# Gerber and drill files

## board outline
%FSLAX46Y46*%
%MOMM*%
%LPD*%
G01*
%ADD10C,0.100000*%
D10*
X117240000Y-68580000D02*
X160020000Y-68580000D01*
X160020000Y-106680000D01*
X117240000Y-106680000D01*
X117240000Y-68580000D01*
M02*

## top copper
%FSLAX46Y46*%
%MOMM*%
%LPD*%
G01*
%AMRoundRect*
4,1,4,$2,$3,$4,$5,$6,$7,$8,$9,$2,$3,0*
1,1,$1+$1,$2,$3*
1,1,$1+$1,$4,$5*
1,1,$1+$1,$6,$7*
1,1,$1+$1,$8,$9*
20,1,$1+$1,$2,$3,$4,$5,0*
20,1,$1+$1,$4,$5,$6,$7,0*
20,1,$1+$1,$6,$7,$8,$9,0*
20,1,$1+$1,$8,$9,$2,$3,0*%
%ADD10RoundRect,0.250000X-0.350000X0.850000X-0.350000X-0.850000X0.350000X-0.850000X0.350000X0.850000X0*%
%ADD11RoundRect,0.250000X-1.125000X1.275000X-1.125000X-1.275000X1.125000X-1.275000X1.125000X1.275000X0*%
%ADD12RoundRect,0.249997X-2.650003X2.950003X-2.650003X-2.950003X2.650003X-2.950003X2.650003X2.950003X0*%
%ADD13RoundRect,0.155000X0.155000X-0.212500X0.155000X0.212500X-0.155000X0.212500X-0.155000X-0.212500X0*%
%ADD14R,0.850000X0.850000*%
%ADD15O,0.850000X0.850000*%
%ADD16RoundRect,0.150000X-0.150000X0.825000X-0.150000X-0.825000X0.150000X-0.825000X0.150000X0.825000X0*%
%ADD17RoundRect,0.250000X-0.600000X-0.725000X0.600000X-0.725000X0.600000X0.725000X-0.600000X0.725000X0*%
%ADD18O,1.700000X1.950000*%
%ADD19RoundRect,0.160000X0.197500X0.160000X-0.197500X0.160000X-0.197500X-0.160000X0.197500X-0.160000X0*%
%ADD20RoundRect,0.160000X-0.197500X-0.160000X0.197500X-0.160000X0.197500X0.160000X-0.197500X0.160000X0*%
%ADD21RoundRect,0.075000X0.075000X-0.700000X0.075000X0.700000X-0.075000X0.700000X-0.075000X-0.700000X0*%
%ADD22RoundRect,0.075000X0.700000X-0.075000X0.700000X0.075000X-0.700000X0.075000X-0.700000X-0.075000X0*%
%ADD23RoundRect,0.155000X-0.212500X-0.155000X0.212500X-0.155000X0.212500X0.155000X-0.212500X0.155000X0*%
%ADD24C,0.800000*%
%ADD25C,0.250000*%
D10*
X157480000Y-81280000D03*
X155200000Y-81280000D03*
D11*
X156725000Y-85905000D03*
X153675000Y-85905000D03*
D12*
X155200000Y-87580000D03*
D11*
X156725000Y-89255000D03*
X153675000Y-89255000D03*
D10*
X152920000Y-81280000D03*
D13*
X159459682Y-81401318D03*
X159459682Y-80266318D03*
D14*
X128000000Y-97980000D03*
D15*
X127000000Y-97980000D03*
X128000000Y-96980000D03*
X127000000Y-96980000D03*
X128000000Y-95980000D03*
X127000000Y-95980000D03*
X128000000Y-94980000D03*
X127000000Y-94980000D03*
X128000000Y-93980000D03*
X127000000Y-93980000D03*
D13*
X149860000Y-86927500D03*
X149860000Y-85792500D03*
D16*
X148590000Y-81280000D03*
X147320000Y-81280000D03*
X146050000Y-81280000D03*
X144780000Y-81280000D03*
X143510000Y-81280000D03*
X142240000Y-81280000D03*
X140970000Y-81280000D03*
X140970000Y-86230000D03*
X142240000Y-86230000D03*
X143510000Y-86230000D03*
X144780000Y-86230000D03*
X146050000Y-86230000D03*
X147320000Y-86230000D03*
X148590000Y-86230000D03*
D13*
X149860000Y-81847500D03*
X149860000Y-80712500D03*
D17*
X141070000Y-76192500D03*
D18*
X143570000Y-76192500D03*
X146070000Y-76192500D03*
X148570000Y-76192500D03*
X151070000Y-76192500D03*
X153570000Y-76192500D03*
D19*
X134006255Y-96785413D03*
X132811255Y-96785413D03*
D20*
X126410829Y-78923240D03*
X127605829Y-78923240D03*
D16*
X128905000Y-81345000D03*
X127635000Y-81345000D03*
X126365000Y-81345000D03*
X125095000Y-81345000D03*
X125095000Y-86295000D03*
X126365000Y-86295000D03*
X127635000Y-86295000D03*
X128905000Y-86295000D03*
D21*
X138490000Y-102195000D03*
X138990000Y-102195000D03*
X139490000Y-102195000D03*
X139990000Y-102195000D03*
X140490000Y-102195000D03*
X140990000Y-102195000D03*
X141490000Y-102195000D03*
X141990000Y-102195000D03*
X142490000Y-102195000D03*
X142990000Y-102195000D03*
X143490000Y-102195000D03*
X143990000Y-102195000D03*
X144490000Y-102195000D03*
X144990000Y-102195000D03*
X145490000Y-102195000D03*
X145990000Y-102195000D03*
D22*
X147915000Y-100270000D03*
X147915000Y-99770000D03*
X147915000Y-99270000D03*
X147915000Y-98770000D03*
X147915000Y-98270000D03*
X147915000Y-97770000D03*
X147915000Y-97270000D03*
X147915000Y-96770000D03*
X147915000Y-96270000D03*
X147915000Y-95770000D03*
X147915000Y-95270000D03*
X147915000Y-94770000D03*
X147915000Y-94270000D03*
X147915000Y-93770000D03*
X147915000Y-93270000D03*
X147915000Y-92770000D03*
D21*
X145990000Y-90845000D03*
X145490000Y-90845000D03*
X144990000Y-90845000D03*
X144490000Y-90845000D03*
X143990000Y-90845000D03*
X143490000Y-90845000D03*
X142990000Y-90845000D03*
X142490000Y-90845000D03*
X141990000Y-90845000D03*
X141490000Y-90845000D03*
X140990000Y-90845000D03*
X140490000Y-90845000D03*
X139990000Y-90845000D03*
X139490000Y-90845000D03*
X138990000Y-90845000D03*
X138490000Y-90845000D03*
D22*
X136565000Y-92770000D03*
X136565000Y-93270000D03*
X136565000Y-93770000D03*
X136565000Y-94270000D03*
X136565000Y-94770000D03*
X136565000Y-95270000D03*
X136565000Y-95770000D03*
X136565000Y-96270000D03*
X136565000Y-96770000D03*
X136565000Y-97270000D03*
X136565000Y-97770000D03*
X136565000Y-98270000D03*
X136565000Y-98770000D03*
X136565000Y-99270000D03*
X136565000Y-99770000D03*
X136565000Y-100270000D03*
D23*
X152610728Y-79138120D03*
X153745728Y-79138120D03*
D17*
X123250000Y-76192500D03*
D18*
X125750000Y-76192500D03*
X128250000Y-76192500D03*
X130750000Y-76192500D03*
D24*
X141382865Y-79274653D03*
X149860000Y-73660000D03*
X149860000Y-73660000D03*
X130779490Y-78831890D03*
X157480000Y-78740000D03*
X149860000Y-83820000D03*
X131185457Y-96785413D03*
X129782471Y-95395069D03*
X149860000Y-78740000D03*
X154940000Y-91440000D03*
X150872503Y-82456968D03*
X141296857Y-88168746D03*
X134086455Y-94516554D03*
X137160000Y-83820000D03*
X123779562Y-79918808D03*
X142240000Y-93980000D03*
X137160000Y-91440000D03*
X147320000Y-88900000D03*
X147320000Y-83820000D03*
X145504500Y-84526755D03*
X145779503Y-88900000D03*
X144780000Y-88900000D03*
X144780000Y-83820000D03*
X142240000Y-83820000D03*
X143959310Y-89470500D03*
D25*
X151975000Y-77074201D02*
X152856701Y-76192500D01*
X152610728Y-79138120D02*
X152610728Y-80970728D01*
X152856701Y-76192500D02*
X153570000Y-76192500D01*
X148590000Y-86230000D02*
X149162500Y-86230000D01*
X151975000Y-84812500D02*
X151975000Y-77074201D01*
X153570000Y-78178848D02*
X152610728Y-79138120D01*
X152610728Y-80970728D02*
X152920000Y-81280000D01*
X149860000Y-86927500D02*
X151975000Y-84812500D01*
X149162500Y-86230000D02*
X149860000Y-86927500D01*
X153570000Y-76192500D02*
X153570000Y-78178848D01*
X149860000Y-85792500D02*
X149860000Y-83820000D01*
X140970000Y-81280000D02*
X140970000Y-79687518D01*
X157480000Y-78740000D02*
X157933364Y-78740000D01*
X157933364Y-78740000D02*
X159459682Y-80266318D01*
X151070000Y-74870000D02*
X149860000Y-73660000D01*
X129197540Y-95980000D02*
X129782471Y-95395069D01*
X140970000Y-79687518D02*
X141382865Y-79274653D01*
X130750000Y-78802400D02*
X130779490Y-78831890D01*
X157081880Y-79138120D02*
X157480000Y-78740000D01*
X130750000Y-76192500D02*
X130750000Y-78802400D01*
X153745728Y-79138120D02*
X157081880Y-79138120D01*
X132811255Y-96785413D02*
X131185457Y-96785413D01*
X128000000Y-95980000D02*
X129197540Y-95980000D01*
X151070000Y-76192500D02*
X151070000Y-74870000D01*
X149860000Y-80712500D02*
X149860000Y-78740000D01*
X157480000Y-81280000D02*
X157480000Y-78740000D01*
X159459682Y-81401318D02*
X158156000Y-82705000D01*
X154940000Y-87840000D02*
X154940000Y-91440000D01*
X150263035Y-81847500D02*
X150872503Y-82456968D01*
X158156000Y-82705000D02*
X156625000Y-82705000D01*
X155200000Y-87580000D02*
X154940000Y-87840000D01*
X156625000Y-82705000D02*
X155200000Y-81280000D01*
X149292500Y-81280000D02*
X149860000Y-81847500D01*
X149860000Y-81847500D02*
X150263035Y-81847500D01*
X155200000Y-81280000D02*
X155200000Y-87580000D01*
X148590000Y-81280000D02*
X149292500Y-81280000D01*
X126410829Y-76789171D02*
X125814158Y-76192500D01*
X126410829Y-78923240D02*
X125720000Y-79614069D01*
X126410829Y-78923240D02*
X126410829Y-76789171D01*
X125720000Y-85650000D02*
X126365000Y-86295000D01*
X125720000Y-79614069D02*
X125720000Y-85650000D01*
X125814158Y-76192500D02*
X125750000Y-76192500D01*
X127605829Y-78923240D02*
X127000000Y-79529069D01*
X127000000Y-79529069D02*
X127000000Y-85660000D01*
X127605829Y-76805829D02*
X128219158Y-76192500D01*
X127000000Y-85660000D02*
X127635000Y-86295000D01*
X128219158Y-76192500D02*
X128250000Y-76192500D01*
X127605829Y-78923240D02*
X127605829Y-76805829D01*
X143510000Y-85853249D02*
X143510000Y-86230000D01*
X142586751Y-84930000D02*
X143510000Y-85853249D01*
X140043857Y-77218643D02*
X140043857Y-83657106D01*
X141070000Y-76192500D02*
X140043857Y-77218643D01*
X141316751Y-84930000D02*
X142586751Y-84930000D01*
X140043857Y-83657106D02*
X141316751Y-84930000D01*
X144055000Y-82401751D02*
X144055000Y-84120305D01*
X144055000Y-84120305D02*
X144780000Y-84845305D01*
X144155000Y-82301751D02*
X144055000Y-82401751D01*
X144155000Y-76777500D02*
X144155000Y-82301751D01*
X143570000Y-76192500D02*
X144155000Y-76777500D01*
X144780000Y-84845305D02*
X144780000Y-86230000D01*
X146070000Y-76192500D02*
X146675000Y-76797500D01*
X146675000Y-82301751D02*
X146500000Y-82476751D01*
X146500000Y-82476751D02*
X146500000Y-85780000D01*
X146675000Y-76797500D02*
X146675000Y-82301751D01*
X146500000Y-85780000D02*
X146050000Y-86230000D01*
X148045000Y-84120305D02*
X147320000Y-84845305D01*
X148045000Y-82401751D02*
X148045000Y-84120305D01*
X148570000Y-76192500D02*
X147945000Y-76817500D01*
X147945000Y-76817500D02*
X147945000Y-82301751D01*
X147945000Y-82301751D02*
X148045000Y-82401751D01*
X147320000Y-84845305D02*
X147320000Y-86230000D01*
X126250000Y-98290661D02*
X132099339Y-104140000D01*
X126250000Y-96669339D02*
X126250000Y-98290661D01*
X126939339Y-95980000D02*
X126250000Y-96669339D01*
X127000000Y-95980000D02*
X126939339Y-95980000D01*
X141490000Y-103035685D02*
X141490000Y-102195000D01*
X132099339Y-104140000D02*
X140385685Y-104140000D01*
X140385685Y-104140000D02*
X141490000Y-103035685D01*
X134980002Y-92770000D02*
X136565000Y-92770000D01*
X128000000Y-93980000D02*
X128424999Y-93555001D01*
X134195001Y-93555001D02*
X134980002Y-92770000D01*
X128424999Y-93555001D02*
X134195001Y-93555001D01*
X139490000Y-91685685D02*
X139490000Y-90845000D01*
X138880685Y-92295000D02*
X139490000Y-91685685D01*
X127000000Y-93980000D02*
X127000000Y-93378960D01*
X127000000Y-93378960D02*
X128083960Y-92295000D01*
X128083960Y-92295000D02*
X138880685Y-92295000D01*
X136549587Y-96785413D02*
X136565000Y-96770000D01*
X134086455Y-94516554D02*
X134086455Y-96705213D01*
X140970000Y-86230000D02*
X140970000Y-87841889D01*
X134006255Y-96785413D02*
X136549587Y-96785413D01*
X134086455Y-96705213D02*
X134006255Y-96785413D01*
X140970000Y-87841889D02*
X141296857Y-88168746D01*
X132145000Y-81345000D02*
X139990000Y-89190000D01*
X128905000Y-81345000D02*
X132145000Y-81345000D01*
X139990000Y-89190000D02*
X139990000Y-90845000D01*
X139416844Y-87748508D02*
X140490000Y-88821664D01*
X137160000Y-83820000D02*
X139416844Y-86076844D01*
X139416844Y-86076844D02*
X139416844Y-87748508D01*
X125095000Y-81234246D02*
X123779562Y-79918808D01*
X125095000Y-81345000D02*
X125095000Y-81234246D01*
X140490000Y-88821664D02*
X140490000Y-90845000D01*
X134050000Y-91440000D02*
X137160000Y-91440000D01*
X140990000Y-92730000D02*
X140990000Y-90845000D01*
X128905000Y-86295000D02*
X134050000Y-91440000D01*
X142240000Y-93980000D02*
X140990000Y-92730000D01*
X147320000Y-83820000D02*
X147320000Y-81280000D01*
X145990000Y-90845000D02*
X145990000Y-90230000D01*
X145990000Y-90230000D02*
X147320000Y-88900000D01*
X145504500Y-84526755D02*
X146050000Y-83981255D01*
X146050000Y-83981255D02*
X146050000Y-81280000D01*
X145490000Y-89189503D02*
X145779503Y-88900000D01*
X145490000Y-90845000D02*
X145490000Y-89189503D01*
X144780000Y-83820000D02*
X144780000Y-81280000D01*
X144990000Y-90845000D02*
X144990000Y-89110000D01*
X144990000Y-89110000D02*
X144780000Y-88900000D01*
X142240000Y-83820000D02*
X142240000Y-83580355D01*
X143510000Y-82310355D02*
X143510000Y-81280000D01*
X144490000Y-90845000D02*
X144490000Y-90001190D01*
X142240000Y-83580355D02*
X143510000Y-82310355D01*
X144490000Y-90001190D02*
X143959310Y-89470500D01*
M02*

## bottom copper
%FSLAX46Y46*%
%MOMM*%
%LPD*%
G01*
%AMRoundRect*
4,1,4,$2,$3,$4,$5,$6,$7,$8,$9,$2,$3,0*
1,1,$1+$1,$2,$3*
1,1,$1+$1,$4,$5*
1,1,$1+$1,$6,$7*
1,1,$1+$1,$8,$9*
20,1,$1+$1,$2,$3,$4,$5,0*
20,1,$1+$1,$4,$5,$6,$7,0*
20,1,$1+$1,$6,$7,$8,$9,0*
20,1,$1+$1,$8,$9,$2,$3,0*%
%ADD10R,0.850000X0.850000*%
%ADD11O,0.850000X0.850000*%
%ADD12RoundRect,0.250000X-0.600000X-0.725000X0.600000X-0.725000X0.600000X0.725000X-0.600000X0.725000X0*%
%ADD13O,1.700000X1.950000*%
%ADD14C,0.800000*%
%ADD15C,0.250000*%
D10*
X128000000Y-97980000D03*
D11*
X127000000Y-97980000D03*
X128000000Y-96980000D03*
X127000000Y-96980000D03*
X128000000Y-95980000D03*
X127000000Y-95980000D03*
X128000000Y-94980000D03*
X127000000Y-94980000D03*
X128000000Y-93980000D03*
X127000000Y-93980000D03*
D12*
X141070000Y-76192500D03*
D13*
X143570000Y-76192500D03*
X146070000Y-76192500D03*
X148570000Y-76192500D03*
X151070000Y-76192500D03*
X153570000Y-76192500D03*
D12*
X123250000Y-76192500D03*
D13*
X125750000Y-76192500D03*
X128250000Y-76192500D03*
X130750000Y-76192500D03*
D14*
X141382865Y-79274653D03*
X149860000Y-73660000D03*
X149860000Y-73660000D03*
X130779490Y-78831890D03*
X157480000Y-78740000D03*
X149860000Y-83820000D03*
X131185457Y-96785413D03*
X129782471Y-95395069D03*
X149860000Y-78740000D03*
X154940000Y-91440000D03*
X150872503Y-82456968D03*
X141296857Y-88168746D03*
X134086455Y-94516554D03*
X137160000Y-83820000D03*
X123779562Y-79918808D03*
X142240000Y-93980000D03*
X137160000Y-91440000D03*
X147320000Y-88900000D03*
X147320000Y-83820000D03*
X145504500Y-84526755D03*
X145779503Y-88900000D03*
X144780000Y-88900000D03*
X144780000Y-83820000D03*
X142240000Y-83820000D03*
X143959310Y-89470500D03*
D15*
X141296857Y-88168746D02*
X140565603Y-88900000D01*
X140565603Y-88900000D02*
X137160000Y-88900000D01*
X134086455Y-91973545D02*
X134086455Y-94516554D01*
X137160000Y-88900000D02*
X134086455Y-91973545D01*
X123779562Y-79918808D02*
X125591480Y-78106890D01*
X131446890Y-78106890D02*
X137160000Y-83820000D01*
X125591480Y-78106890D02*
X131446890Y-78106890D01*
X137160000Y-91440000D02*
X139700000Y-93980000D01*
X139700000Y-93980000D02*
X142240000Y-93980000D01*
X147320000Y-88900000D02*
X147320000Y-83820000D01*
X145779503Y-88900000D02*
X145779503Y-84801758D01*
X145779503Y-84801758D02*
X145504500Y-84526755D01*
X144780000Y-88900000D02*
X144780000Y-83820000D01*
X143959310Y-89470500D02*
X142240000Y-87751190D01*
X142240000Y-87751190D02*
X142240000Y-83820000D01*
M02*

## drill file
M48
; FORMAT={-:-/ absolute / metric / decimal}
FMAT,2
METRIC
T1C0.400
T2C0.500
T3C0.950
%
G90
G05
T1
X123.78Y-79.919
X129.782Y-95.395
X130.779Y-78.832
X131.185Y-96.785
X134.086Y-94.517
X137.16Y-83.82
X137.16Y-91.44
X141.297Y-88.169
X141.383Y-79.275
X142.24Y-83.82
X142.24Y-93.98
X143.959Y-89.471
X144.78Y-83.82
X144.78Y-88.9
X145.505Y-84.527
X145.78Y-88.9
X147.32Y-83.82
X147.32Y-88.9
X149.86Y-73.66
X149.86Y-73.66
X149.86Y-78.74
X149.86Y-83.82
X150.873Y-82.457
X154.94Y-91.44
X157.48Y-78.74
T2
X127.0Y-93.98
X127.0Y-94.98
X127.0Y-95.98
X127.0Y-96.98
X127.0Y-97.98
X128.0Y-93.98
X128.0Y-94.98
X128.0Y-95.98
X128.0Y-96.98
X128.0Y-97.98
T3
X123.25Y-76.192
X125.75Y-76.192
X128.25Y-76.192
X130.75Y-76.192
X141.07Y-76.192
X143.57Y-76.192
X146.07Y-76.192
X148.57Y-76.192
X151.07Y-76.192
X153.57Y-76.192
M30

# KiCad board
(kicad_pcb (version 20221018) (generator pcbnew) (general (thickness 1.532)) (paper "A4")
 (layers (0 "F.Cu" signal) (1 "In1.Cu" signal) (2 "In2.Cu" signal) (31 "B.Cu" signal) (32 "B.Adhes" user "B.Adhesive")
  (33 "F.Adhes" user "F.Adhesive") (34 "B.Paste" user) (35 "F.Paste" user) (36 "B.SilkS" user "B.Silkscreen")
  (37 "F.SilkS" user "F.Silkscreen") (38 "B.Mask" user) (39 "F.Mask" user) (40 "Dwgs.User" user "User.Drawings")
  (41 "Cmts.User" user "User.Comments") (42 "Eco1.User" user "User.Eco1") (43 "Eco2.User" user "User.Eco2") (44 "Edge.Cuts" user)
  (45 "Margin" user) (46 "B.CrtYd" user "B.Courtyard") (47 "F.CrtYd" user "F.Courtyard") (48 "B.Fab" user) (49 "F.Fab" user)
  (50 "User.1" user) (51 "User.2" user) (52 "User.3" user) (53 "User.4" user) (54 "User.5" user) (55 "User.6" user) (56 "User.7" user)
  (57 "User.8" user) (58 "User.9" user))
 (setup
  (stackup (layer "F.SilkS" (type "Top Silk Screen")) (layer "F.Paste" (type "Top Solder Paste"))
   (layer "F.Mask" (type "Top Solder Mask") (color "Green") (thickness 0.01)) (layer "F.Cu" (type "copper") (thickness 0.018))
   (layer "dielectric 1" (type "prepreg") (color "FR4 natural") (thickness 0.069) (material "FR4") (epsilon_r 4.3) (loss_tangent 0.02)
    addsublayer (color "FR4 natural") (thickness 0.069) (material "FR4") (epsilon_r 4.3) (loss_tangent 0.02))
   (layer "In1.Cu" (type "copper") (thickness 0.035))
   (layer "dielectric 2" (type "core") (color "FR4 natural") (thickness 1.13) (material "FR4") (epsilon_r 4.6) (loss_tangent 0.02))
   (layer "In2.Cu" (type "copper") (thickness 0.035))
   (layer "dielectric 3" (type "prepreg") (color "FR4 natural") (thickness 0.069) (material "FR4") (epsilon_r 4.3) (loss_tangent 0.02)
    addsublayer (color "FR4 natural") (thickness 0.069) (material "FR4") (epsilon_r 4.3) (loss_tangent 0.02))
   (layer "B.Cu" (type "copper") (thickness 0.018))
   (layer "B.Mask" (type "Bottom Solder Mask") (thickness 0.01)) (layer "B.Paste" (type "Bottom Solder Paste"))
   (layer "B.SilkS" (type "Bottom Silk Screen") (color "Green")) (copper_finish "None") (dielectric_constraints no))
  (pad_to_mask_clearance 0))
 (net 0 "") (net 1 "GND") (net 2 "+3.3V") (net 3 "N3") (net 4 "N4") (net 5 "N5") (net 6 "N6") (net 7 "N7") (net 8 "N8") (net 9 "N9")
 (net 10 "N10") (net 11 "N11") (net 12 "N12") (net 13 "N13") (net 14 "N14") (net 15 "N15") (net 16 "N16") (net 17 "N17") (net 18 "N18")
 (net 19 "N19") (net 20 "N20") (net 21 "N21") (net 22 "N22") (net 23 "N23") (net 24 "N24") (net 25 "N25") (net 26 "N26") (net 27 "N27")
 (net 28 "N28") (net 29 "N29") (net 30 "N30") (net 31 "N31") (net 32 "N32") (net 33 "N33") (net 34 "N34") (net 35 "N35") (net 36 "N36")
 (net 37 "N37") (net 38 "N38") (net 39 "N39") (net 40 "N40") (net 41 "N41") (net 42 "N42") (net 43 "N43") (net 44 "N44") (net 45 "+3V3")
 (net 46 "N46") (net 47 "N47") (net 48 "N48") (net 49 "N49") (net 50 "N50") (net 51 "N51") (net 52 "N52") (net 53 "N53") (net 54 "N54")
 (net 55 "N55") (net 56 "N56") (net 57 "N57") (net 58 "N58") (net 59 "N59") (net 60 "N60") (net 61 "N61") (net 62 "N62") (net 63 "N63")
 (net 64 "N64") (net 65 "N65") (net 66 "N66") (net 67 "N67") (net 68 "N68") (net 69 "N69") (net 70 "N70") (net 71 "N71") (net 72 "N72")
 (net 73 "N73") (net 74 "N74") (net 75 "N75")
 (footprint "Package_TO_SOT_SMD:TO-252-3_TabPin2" (layer "F.Cu") (at 155.2 86.32 -90)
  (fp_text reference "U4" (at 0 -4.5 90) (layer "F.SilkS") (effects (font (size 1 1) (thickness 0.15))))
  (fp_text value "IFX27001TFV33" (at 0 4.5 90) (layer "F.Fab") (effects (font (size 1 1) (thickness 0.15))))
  (pad "1" smd roundrect (at -5.04 -2.28 270) (size 2.2 1.2) (layers "F.Cu" "F.Paste" "F.Mask") (roundrect_rratio 0.208333) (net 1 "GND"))
  (pad "2" smd roundrect (at -5.04 0 270) (size 2.2 1.2) (layers "F.Cu" "F.Paste" "F.Mask") (roundrect_rratio 0.208333) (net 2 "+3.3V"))
  (pad "2" smd roundrect (at -0.415 -1.525 270) (size 3.05 2.75) (layers "F.Cu" "F.Paste") (roundrect_rratio 0.090909) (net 2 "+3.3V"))
  (pad "2" smd roundrect (at -0.415 1.525 270) (size 3.05 2.75) (layers "F.Cu" "F.Paste") (roundrect_rratio 0.090909) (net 2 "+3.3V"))
  (pad "2" smd roundrect (at 1.26 0 270) (size 6.4 5.8) (layers "F.Cu" "F.Mask") (roundrect_rratio 0.043103) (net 2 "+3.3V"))
  (pad "2" smd roundrect (at 2.935 -1.525 270) (size 3.05 2.75) (layers "F.Cu" "F.Paste") (roundrect_rratio 0.090909) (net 2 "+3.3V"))
  (pad "2" smd roundrect (at 2.935 1.525 270) (size 3.05 2.75) (layers "F.Cu" "F.Paste") (roundrect_rratio 0.090909) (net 2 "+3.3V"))
  (pad "3" smd roundrect (at -5.04 2.28 270) (size 2.2 1.2) (layers "F.Cu" "F.Paste" "F.Mask") (roundrect_rratio 0.208333) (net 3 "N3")))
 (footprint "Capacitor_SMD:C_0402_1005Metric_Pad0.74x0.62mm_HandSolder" (layer "F.Cu") (at 159.459682 80.833818 90)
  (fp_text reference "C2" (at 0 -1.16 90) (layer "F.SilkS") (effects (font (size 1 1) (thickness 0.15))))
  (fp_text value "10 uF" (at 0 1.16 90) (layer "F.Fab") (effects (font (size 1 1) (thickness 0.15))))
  (pad "1" smd roundrect (at -0.5675 0 90) (size 0.735 0.62) (layers "F.Cu" "F.Paste" "F.Mask") (roundrect_rratio 0.25) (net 2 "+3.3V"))
  (pad "2" smd roundrect (at 0.5675 0 90) (size 0.735 0.62) (layers "F.Cu" "F.Paste" "F.Mask") (roundrect_rratio 0.25) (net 1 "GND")))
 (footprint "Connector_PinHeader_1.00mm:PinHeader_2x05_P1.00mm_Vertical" (layer "F.Cu") (at 128 97.98 180)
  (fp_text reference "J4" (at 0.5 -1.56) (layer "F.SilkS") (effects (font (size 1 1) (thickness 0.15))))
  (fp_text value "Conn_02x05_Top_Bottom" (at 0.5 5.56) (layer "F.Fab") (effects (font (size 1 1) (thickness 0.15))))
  (pad "1" thru_hole rect (at 0 0 180) (size 0.85 0.85) (drill 0.5) (layers "*.Cu" "*.Mask") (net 2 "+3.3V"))
  (pad "2" thru_hole oval (at 1 0 180) (size 0.85 0.85) (drill 0.5) (layers "*.Cu" "*.Mask") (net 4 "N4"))
  (pad "3" thru_hole oval (at 0 1 180) (size 0.85 0.85) (drill 0.5) (layers "*.Cu" "*.Mask") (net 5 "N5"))
  (pad "4" thru_hole oval (at 1 1 180) (size 0.85 0.85) (drill 0.5) (layers "*.Cu" "*.Mask") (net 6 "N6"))
  (pad "5" thru_hole oval (at 0 2 180) (size 0.85 0.85) (drill 0.5) (layers "*.Cu" "*.Mask") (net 1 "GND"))
  (pad "6" thru_hole oval (at 1 2 180) (size 0.85 0.85) (drill 0.5) (layers "*.Cu" "*.Mask") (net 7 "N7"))
  (pad "7" thru_hole oval (at 0 3 180) (size 0.85 0.85) (drill 0.5) (layers "*.Cu" "*.Mask") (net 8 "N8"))
  (pad "8" thru_hole oval (at 1 3 180) (size 0.85 0.85) (drill 0.5) (layers "*.Cu" "*.Mask") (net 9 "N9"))
  (pad "9" thru_hole oval (at 0 4 180) (size 0.85 0.85) (drill 0.5) (layers "*.Cu" "*.Mask") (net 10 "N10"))
  (pad "10" thru_hole oval (at 1 4 180) (size 0.85 0.85) (drill 0.5) (layers "*.Cu" "*.Mask") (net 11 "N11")))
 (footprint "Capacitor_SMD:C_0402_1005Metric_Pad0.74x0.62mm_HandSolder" (layer "F.Cu") (at 149.86 86.36 90)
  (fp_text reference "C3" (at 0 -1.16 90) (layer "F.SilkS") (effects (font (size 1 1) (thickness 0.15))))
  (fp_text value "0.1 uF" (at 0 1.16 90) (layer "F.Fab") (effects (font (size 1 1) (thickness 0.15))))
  (pad "1" smd roundrect (at -0.5675 0 90) (size 0.735 0.62) (layers "F.Cu" "F.Paste" "F.Mask") (roundrect_rratio 0.25) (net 3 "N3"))
  (pad "2" smd roundrect (at 0.5675 0 90) (size 0.735 0.62) (layers "F.Cu" "F.Paste" "F.Mask") (roundrect_rratio 0.25) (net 1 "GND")))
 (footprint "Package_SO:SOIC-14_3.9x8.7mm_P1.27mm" (layer "F.Cu") (at 144.78 83.755 -90)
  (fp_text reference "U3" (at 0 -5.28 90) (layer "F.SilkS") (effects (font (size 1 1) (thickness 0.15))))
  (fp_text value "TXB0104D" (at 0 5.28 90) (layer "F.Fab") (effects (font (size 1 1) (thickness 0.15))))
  (pad "1" smd roundrect (at -2.475 -3.81 270) (size 1.95 0.6) (layers "F.Cu" "F.Paste" "F.Mask") (roundrect_rratio 0.25) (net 2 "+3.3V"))
  (pad "2" smd roundrect (at -2.475 -2.54 270) (size 1.95 0.6) (layers "F.Cu" "F.Paste" "F.Mask") (roundrect_rratio 0.25) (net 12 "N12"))
  (pad "3" smd roundrect (at -2.475 -1.27 270) (size 1.95 0.6) (layers "F.Cu" "F.Paste" "F.Mask") (roundrect_rratio 0.25) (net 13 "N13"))
  (pad "4" smd roundrect (at -2.475 0 270) (size 1.95 0.6) (layers "F.Cu" "F.Paste" "F.Mask") (roundrect_rratio 0.25) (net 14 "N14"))
  (pad "5" smd roundrect (at -2.475 1.27 270) (size 1.95 0.6) (layers "F.Cu" "F.Paste" "F.Mask") (roundrect_rratio 0.25) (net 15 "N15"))
  (pad "6" smd roundrect (at -2.475 2.54 270) (size 1.95 0.6) (layers "F.Cu" "F.Paste" "F.Mask") (roundrect_rratio 0.25) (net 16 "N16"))
  (pad "7" smd roundrect (at -2.475 3.81 270) (size 1.95 0.6) (layers "F.Cu" "F.Paste" "F.Mask") (roundrect_rratio 0.25) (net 1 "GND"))
  (pad "8" smd roundrect (at 2.475 3.81 270) (size 1.95 0.6) (layers "F.Cu" "F.Paste" "F.Mask") (roundrect_rratio 0.25) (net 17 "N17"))
  (pad "9" smd roundrect (at 2.475 2.54 270) (size 1.95 0.6) (layers "F.Cu" "F.Paste" "F.Mask") (roundrect_rratio 0.25) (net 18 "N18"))
  (pad "10" smd roundrect (at 2.475 1.27 270) (size 1.95 0.6) (layers "F.Cu" "F.Paste" "F.Mask") (roundrect_rratio 0.25) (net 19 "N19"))
  (pad "11" smd roundrect (at 2.475 0 270) (size 1.95 0.6) (layers "F.Cu" "F.Paste" "F.Mask") (roundrect_rratio 0.25) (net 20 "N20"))
  (pad "12" smd roundrect (at 2.475 -1.27 270) (size 1.95 0.6) (layers "F.Cu" "F.Paste" "F.Mask") (roundrect_rratio 0.25) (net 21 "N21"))
  (pad "13" smd roundrect (at 2.475 -2.54 270) (size 1.95 0.6) (layers "F.Cu" "F.Paste" "F.Mask") (roundrect_rratio 0.25) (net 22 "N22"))
  (pad "14" smd roundrect (at 2.475 -3.81 270) (size 1.95 0.6) (layers "F.Cu" "F.Paste" "F.Mask") (roundrect_rratio 0.25) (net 3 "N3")))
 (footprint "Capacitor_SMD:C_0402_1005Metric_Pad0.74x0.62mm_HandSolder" (layer "F.Cu") (at 149.86 81.28 90)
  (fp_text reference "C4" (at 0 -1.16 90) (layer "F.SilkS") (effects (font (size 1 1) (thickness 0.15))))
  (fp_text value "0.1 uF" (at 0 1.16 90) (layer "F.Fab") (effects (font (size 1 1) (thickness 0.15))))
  (pad "1" smd roundrect (at -0.5675 0 90) (size 0.735 0.62) (layers "F.Cu" "F.Paste" "F.Mask") (roundrect_rratio 0.25) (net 2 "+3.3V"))
  (pad "2" smd roundrect (at 0.5675 0 90) (size 0.735 0.62) (layers "F.Cu" "F.Paste" "F.Mask") (roundrect_rratio 0.25) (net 1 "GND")))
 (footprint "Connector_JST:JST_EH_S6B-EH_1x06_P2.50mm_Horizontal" (layer "F.Cu") (at 141.07 76.1925)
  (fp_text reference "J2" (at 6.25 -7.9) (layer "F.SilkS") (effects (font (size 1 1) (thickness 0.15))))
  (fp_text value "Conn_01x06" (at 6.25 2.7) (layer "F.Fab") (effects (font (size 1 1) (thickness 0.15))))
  (pad "1" thru_hole roundrect (at 0 0) (size 1.7 1.95) (drill 0.95) (layers "*.Cu" "*.Mask") (roundrect_rratio 0.147059) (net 19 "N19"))
  (pad "2" thru_hole oval (at 2.5 0) (size 1.7 1.95) (drill 0.95) (layers "*.Cu" "*.Mask") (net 20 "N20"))
  (pad "3" thru_hole oval (at 5 0) (size 1.7 1.95) (drill 0.95) (layers "*.Cu" "*.Mask") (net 21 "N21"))
  (pad "4" thru_hole oval (at 7.5 0) (size 1.7 1.95) (drill 0.95) (layers "*.Cu" "*.Mask") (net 22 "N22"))
  (pad "5" thru_hole oval (at 10 0) (size 1.7 1.95) (drill 0.95) (layers "*.Cu" "*.Mask") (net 1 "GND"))
  (pad "6" thru_hole oval (at 12.5 0) (size 1.7 1.95) (drill 0.95) (layers "*.Cu" "*.Mask") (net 3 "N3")))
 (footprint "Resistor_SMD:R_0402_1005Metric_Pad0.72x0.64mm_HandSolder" (layer "F.Cu") (at 133.408755 96.785413 180)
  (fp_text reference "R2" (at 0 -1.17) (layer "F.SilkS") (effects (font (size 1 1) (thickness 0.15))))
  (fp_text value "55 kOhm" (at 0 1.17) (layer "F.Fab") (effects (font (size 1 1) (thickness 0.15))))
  (pad "1" smd roundrect (at -0.5975 0 180) (size 0.715 0.64) (layers "F.Cu" "F.Paste" "F.Mask") (roundrect_rratio 0.25) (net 17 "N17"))
  (pad "2" smd roundrect (at 0.5975 0 180) (size 0.715 0.64) (layers "F.Cu" "F.Paste" "F.Mask") (roundrect_rratio 0.25) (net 1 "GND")))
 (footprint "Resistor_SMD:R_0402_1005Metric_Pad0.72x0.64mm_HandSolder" (layer "F.Cu") (at 127.008329 78.92324)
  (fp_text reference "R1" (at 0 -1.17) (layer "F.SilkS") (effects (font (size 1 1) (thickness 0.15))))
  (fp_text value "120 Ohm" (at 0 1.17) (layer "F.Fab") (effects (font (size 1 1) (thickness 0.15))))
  (pad "1" smd roundrect (at -0.5975 0) (size 0.715 0.64) (layers "F.Cu" "F.Paste" "F.Mask") (roundrect_rratio 0.25) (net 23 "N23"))
  (pad "2" smd roundrect (at 0.5975 0) (size 0.715 0.64) (layers "F.Cu" "F.Paste" "F.Mask") (roundrect_rratio 0.25) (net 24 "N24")))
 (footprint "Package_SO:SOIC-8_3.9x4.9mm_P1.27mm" (layer "F.Cu") (at 127 83.82 -90)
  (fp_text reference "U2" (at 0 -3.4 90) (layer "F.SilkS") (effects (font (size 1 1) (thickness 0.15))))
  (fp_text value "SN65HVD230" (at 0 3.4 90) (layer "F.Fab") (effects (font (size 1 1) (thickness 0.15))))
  (pad "1" smd roundrect (at -2.475 -1.905 270) (size 1.95 0.6) (layers "F.Cu" "F.Paste" "F.Mask") (roundrect_rratio 0.25) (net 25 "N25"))
  (pad "2" smd roundrect (at -2.475 -0.635 270) (size 1.95 0.6) (layers "F.Cu" "F.Paste" "F.Mask") (roundrect_rratio 0.25) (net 1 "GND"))
  (pad "3" smd roundrect (at -2.475 0.635 270) (size 1.95 0.6) (layers "F.Cu" "F.Paste" "F.Mask") (roundrect_rratio 0.25) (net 2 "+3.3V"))
  (pad "4" smd roundrect (at -2.475 1.905 270) (size 1.95 0.6) (layers "F.Cu" "F.Paste" "F.Mask") (roundrect_rratio 0.25) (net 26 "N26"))
  (pad "5" smd roundrect (at 2.475 1.905 270) (size 1.95 0.6) (layers "F.Cu" "F.Paste" "F.Mask") (roundrect_rratio 0.25) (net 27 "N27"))
  (pad "6" smd roundrect (at 2.475 0.635 270) (size 1.95 0.6) (layers "F.Cu" "F.Paste" "F.Mask") (roundrect_rratio 0.25) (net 23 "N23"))
  (pad "7" smd roundrect (at 2.475 -0.635 270) (size 1.95 0.6) (layers "F.Cu" "F.Paste" "F.Mask") (roundrect_rratio 0.25) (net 24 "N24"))
  (pad "8" smd roundrect (at 2.475 -1.905 270) (size 1.95 0.6) (layers "F.Cu" "F.Paste" "F.Mask") (roundrect_rratio 0.25) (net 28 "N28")))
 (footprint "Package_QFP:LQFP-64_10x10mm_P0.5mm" (layer "F.Cu") (at 142.24 96.52 90)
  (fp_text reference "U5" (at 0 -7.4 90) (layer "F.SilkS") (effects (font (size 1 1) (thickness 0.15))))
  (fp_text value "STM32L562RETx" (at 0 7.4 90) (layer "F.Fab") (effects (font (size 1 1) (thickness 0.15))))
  (pad "1" smd roundrect (at -5.675 -3.75 90) (size 1.55 0.3) (layers "F.Cu" "F.Paste" "F.Mask") (roundrect_rratio 0.25) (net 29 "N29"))
  (pad "2" smd roundrect (at -5.675 -3.25 90) (size 1.55 0.3) (layers "F.Cu" "F.Paste" "F.Mask") (roundrect_rratio 0.25) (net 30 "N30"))
  (pad "3" smd roundrect (at -5.675 -2.75 90) (size 1.55 0.3) (layers "F.Cu" "F.Paste" "F.Mask") (roundrect_rratio 0.25) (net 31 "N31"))
  (pad "4" smd roundrect (at -5.675 -2.25 90) (size 1.55 0.3) (layers "F.Cu" "F.Paste" "F.Mask") (roundrect_rratio 0.25) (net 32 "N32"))
  (pad "5" smd roundrect (at -5.675 -1.75 90) (size 1.55 0.3) (layers "F.Cu" "F.Paste" "F.Mask") (roundrect_rratio 0.25) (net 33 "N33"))
  (pad "6" smd roundrect (at -5.675 -1.25 90) (size 1.55 0.3) (layers "F.Cu" "F.Paste" "F.Mask") (roundrect_rratio 0.25) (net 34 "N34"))
  (pad "7" smd roundrect (at -5.675 -0.75 90) (size 1.55 0.3) (layers "F.Cu" "F.Paste" "F.Mask") (roundrect_rratio 0.25) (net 7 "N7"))
  (pad "8" smd roundrect (at -5.675 -0.25 90) (size 1.55 0.3) (layers "F.Cu" "F.Paste" "F.Mask") (roundrect_rratio 0.25) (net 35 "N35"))
  (pad "9" smd roundrect (at -5.675 0.25 90) (size 1.55 0.3) (layers "F.Cu" "F.Paste" "F.Mask") (roundrect_rratio 0.25) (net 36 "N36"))
  (pad "10" smd roundrect (at -5.675 0.75 90) (size 1.55 0.3) (layers "F.Cu" "F.Paste" "F.Mask") (roundrect_rratio 0.25) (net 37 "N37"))
  (pad "11" smd roundrect (at -5.675 1.25 90) (size 1.55 0.3) (layers "F.Cu" "F.Paste" "F.Mask") (roundrect_rratio 0.25) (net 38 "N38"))
  (pad "12" smd roundrect (at -5.675 1.75 90) (size 1.55 0.3) (layers "F.Cu" "F.Paste" "F.Mask") (roundrect_rratio 0.25) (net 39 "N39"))
  (pad "13" smd roundrect (at -5.675 2.25 90) (size 1.55 0.3) (layers "F.Cu" "F.Paste" "F.Mask") (roundrect_rratio 0.25) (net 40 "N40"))
  (pad "14" smd roundrect (at -5.675 2.75 90) (size 1.55 0.3) (layers "F.Cu" "F.Paste" "F.Mask") (roundrect_rratio 0.25) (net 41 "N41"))
  (pad "15" smd roundrect (at -5.675 3.25 90) (size 1.55 0.3) (layers "F.Cu" "F.Paste" "F.Mask") (roundrect_rratio 0.25) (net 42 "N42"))
  (pad "16" smd roundrect (at -5.675 3.75 90) (size 1.55 0.3) (layers "F.Cu" "F.Paste" "F.Mask") (roundrect_rratio 0.25) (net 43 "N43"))
  (pad "17" smd roundrect (at -3.75 5.675 90) (size 0.3 1.55) (layers "F.Cu" "F.Paste" "F.Mask") (roundrect_rratio 0.25) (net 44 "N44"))
  (pad "18" smd roundrect (at -3.25 5.675 90) (size 0.3 1.55) (layers "F.Cu" "F.Paste" "F.Mask") (roundrect_rratio 0.25) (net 1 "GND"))
  (pad "19" smd roundrect (at -2.75 5.675 90) (size 0.3 1.55) (layers "F.Cu" "F.Paste" "F.Mask") (roundrect_rratio 0.25) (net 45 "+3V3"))
  (pad "20" smd roundrect (at -2.25 5.675 90) (size 0.3 1.55) (layers "F.Cu" "F.Paste" "F.Mask") (roundrect_rratio 0.25) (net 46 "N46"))
  (pad "21" smd roundrect (at -1.75 5.675 90) (size 0.3 1.55) (layers "F.Cu" "F.Paste" "F.Mask") (roundrect_rratio 0.25) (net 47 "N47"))
  (pad "22" smd roundrect (at -1.25 5.675 90) (size 0.3 1.55) (layers "F.Cu" "F.Paste" "F.Mask") (roundrect_rratio 0.25) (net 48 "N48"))
  (pad "23" smd roundrect (at -0.75 5.675 90) (size 0.3 1.55) (layers "F.Cu" "F.Paste" "F.Mask") (roundrect_rratio 0.25) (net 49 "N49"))
  (pad "24" smd roundrect (at -0.25 5.675 90) (size 0.3 1.55) (layers "F.Cu" "F.Paste" "F.Mask") (roundrect_rratio 0.25) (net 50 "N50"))
  (pad "25" smd roundrect (at 0.25 5.675 90) (size 0.3 1.55) (layers "F.Cu" "F.Paste" "F.Mask") (roundrect_rratio 0.25) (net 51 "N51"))
  (pad "26" smd roundrect (at 0.75 5.675 90) (size 0.3 1.55) (layers "F.Cu" "F.Paste" "F.Mask") (roundrect_rratio 0.25) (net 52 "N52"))
  (pad "27" smd roundrect (at 1.25 5.675 90) (size 0.3 1.55) (layers "F.Cu" "F.Paste" "F.Mask") (roundrect_rratio 0.25) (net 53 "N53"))
  (pad "28" smd roundrect (at 1.75 5.675 90) (size 0.3 1.55) (layers "F.Cu" "F.Paste" "F.Mask") (roundrect_rratio 0.25) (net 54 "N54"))
  (pad "29" smd roundrect (at 2.25 5.675 90) (size 0.3 1.55) (layers "F.Cu" "F.Paste" "F.Mask") (roundrect_rratio 0.25) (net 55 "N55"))
  (pad "30" smd roundrect (at 2.75 5.675 90) (size 0.3 1.55) (layers "F.Cu" "F.Paste" "F.Mask") (roundrect_rratio 0.25) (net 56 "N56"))
  (pad "31" smd roundrect (at 3.25 5.675 90) (size 0.3 1.55) (layers "F.Cu" "F.Paste" "F.Mask") (roundrect_rratio 0.25) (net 1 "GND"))
  (pad "32" smd roundrect (at 3.75 5.675 90) (size 0.3 1.55) (layers "F.Cu" "F.Paste" "F.Mask") (roundrect_rratio 0.25) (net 45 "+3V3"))
  (pad "33" smd roundrect (at 5.675 3.75 90) (size 1.55 0.3) (layers "F.Cu" "F.Paste" "F.Mask") (roundrect_rratio 0.25) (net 12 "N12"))
  (pad "34" smd roundrect (at 5.675 3.25 90) (size 1.55 0.3) (layers "F.Cu" "F.Paste" "F.Mask") (roundrect_rratio 0.25) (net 13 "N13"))
  (pad "35" smd roundrect (at 5.675 2.75 90) (size 1.55 0.3) (layers "F.Cu" "F.Paste" "F.Mask") (roundrect_rratio 0.25) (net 14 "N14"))
  (pad "36" smd roundrect (at 5.675 2.25 90) (size 1.55 0.3) (layers "F.Cu" "F.Paste" "F.Mask") (roundrect_rratio 0.25) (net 15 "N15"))
  (pad "37" smd roundrect (at 5.675 1.75 90) (size 1.55 0.3) (layers "F.Cu" "F.Paste" "F.Mask") (roundrect_rratio 0.25) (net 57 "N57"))
  (pad "38" smd roundrect (at 5.675 1.25 90) (size 1.55 0.3) (layers "F.Cu" "F.Paste" "F.Mask") (roundrect_rratio 0.25) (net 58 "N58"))
  (pad "39" smd roundrect (at 5.675 0.75 90) (size 1.55 0.3) (layers "F.Cu" "F.Paste" "F.Mask") (roundrect_rratio 0.25) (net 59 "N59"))
  (pad "40" smd roundrect (at 5.675 0.25 90) (size 1.55 0.3) (layers "F.Cu" "F.Paste" "F.Mask") (roundrect_rratio 0.25) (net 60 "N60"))
  (pad "41" smd roundrect (at 5.675 -0.25 90) (size 1.55 0.3) (layers "F.Cu" "F.Paste" "F.Mask") (roundrect_rratio 0.25) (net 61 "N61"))
  (pad "42" smd roundrect (at 5.675 -0.75 90) (size 1.55 0.3) (layers "F.Cu" "F.Paste" "F.Mask") (roundrect_rratio 0.25) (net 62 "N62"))
  (pad "43" smd roundrect (at 5.675 -1.25 90) (size 1.55 0.3) (layers "F.Cu" "F.Paste" "F.Mask") (roundrect_rratio 0.25) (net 28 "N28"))
  (pad "44" smd roundrect (at 5.675 -1.75 90) (size 1.55 0.3) (layers "F.Cu" "F.Paste" "F.Mask") (roundrect_rratio 0.25) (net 26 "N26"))
  (pad "45" smd roundrect (at 5.675 -2.25 90) (size 1.55 0.3) (layers "F.Cu" "F.Paste" "F.Mask") (roundrect_rratio 0.25) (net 25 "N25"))
  (pad "46" smd roundrect (at 5.675 -2.75 90) (size 1.55 0.3) (layers "F.Cu" "F.Paste" "F.Mask") (roundrect_rratio 0.25) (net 11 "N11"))
  (pad "47" smd roundrect (at 5.675 -3.25 90) (size 1.55 0.3) (layers "F.Cu" "F.Paste" "F.Mask") (roundrect_rratio 0.25) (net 1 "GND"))
  (pad "48" smd roundrect (at 5.675 -3.75 90) (size 1.55 0.3) (layers "F.Cu" "F.Paste" "F.Mask") (roundrect_rratio 0.25) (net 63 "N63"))
  (pad "49" smd roundrect (at 3.75 -5.675 90) (size 0.3 1.55) (layers "F.Cu" "F.Paste" "F.Mask") (roundrect_rratio 0.25) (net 10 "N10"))
  (pad "50" smd roundrect (at 3.25 -5.675 90) (size 0.3 1.55) (layers "F.Cu" "F.Paste" "F.Mask") (roundrect_rratio 0.25) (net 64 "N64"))
  (pad "51" smd roundrect (at 2.75 -5.675 90) (size 0.3 1.55) (layers "F.Cu" "F.Paste" "F.Mask") (roundrect_rratio 0.25) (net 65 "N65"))
  (pad "52" smd roundrect (at 2.25 -5.675 90) (size 0.3 1.55) (layers "F.Cu" "F.Paste" "F.Mask") (roundrect_rratio 0.25) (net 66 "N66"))
  (pad "53" smd roundrect (at 1.75 -5.675 90) (size 0.3 1.55) (layers "F.Cu" "F.Paste" "F.Mask") (roundrect_rratio 0.25) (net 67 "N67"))
  (pad "54" smd roundrect (at 1.25 -5.675 90) (size 0.3 1.55) (layers "F.Cu" "F.Paste" "F.Mask") (roundrect_rratio 0.25) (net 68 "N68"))
  (pad "55" smd roundrect (at 0.75 -5.675 90) (size 0.3 1.55) (layers "F.Cu" "F.Paste" "F.Mask") (roundrect_rratio 0.25) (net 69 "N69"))
  (pad "56" smd roundrect (at 0.25 -5.675 90) (size 0.3 1.55) (layers "F.Cu" "F.Paste" "F.Mask") (roundrect_rratio 0.25) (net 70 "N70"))
  (pad "57" smd roundrect (at -0.25 -5.675 90) (size 0.3 1.55) (layers "F.Cu" "F.Paste" "F.Mask") (roundrect_rratio 0.25) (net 17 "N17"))
  (pad "58" smd roundrect (at -0.75 -5.675 90) (size 0.3 1.55) (layers "F.Cu" "F.Paste" "F.Mask") (roundrect_rratio 0.25) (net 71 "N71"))
  (pad "59" smd roundrect (at -1.25 -5.675 90) (size 0.3 1.55) (layers "F.Cu" "F.Paste" "F.Mask") (roundrect_rratio 0.25) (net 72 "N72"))
  (pad "60" smd roundrect (at -1.75 -5.675 90) (size 0.3 1.55) (layers "F.Cu" "F.Paste" "F.Mask") (roundrect_rratio 0.25) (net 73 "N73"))
  (pad "61" smd roundrect (at -2.25 -5.675 90) (size 0.3 1.55) (layers "F.Cu" "F.Paste" "F.Mask") (roundrect_rratio 0.25) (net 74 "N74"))
  (pad "62" smd roundrect (at -2.75 -5.675 90) (size 0.3 1.55) (layers "F.Cu" "F.Paste" "F.Mask") (roundrect_rratio 0.25) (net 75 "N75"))
  (pad "63" smd roundrect (at -3.25 -5.675 90) (size 0.3 1.55) (layers "F.Cu" "F.Paste" "F.Mask") (roundrect_rratio 0.25) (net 1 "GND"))
  (pad "64" smd roundrect (at -3.75 -5.675 90) (size 0.3 1.55) (layers "F.Cu" "F.Paste" "F.Mask") (roundrect_rratio 0.25) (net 45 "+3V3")))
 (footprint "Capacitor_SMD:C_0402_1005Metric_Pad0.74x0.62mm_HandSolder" (layer "F.Cu") (at 153.178228 79.13812)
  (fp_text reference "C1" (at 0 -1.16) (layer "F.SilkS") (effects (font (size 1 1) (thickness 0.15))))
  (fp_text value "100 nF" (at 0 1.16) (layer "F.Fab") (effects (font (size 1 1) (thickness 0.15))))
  (pad "1" smd roundrect (at -0.5675 0) (size 0.735 0.62) (layers "F.Cu" "F.Paste" "F.Mask") (roundrect_rratio 0.25) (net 3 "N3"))
  (pad "2" smd roundrect (at 0.5675 0) (size 0.735 0.62) (layers "F.Cu" "F.Paste" "F.Mask") (roundrect_rratio 0.25) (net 1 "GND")))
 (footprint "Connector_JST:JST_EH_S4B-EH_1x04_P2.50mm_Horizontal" (layer "F.Cu") (at 123.25 76.1925)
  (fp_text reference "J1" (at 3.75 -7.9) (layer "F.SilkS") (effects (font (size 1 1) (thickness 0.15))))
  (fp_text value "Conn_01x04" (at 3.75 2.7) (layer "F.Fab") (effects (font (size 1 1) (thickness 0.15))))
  (pad "1" thru_hole roundrect (at 0 0) (size 1.7 1.95) (drill 0.95) (layers "*.Cu" "*.Mask") (roundrect_rratio 0.147059) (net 2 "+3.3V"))
  (pad "2" thru_hole oval (at 2.5 0) (size 1.7 1.95) (drill 0.95) (layers "*.Cu" "*.Mask") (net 23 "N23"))
  (pad "3" thru_hole oval (at 5 0) (size 1.7 1.95) (drill 0.95) (layers "*.Cu" "*.Mask") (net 24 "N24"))
  (pad "4" thru_hole oval (at 7.5 0) (size 1.7 1.95) (drill 0.95) (layers "*.Cu" "*.Mask") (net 1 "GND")))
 (gr_rect (start 117.24 68.58) (end 160.02 106.68) (stroke (width 0.1) (type default)) (fill none) (layer "Edge.Cuts"))
 (segment (start 151.975 77.074201) (end 152.856701 76.1925) (width 0.25) (layer "F.Cu") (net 3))
 (segment (start 152.610728 79.13812) (end 152.610728 80.970728) (width 0.25) (layer "F.Cu") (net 3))
 (segment (start 152.856701 76.1925) (end 153.57 76.1925) (width 0.25) (layer "F.Cu") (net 3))
 (segment (start 148.59 86.23) (end 149.1625 86.23) (width 0.25) (layer "F.Cu") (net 3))
 (segment (start 151.975 84.8125) (end 151.975 77.074201) (width 0.25) (layer "F.Cu") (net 3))
 (segment (start 153.57 78.178848) (end 152.610728 79.13812) (width 0.25) (layer "F.Cu") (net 3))
 (segment (start 152.610728 80.970728) (end 152.92 81.28) (width 0.25) (layer "F.Cu") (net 3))
 (segment (start 149.86 86.9275) (end 151.975 84.8125) (width 0.25) (layer "F.Cu") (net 3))
 (segment (start 149.1625 86.23) (end 149.86 86.9275) (width 0.25) (layer "F.Cu") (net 3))
 (segment (start 153.57 76.1925) (end 153.57 78.178848) (width 0.25) (layer "F.Cu") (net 3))
 (segment (start 149.86 85.7925) (end 149.86 83.82) (width 0.25) (layer "F.Cu") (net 1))
 (segment (start 140.97 81.28) (end 140.97 79.687518) (width 0.25) (layer "F.Cu") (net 1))
 (segment (start 157.48 78.74) (end 157.933364 78.74) (width 0.25) (layer "F.Cu") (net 1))
 (segment (start 157.933364 78.74) (end 159.459682 80.266318) (width 0.25) (layer "F.Cu") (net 1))
 (segment (start 151.07 74.87) (end 149.86 73.66) (width 0.25) (layer "F.Cu") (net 1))
 (segment (start 129.19754 95.98) (end 129.782471 95.395069) (width 0.25) (layer "F.Cu") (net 1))
 (segment (start 140.97 79.687518) (end 141.382865 79.274653) (width 0.25) (layer "F.Cu") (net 1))
 (segment (start 130.75 78.8024) (end 130.77949 78.83189) (width 0.25) (layer "F.Cu") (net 1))
 (segment (start 157.08188 79.13812) (end 157.48 78.74) (width 0.25) (layer "F.Cu") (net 1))
 (segment (start 130.75 76.1925) (end 130.75 78.8024) (width 0.25) (layer "F.Cu") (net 1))
 (segment (start 153.745728 79.13812) (end 157.08188 79.13812) (width 0.25) (layer "F.Cu") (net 1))
 (segment (start 132.811255 96.785413) (end 131.185457 96.785413) (width 0.25) (layer "F.Cu") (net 1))
 (segment (start 128 95.98) (end 129.19754 95.98) (width 0.25) (layer "F.Cu") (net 1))
 (segment (start 151.07 76.1925) (end 151.07 74.87) (width 0.25) (layer "F.Cu") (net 1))
 (segment (start 149.86 80.7125) (end 149.86 78.74) (width 0.25) (layer "F.Cu") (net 1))
 (segment (start 157.48 81.28) (end 157.48 78.74) (width 0.25) (layer "F.Cu") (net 1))
 (via (at 141.382865 79.274653) (size 0.8) (drill 0.4) (layers "F.Cu" "B.Cu") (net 1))
 (via (at 149.86 73.66) (size 0.8) (drill 0.4) (layers "F.Cu" "B.Cu") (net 1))
 (via (at 149.86 73.66) (size 0.8) (drill 0.4) (layers "F.Cu" "B.Cu") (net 1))
 (via (at 130.77949 78.83189) (size 0.8) (drill 0.4) (layers "F.Cu" "B.Cu") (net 1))
 (via (at 157.48 78.74) (size 0.8) (drill 0.4) (layers "F.Cu" "B.Cu") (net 1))
 (via (at 149.86 83.82) (size 0.8) (drill 0.4) (layers "F.Cu" "B.Cu") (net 1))
 (via (at 131.185457 96.785413) (size 0.8) (drill 0.4) (layers "F.Cu" "B.Cu") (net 1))
 (via (at 129.782471 95.395069) (size 0.8) (drill 0.4) (layers "F.Cu" "B.Cu") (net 1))
 (via (at 149.86 78.74) (size 0.8) (drill 0.4) (layers "F.Cu" "B.Cu") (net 1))
 (segment (start 159.459682 81.401318) (end 158.156 82.705) (width 0.25) (layer "F.Cu") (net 2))
 (segment (start 154.94 87.84) (end 154.94 91.44) (width 0.25) (layer "F.Cu") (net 2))
 (segment (start 150.263035 81.8475) (end 150.872503 82.456968) (width 0.25) (layer "F.Cu") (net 2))
 (segment (start 158.156 82.705) (end 156.625 82.705) (width 0.25) (layer "F.Cu") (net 2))
 (segment (start 155.2 87.58) (end 154.94 87.84) (width 0.25) (layer "F.Cu") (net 2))
 (segment (start 156.625 82.705) (end 155.2 81.28) (width 0.25) (layer "F.Cu") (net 2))
 (segment (start 149.2925 81.28) (end 149.86 81.8475) (width 0.25) (layer "F.Cu") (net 2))
 (segment (start 149.86 81.8475) (end 150.263035 81.8475) (width 0.25) (layer "F.Cu") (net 2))
 (segment (start 155.2 81.28) (end 155.2 87.58) (width 0.25) (layer "F.Cu") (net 2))
 (segment (start 148.59 81.28) (end 149.2925 81.28) (width 0.25) (layer "F.Cu") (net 2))
 (via (at 154.94 91.44) (size 0.8) (drill 0.4) (layers "F.Cu" "B.Cu") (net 2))
 (via (at 150.872503 82.456968) (size 0.8) (drill 0.4) (layers "F.Cu" "B.Cu") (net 2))
 (segment (start 126.410829 76.789171) (end 125.814158 76.1925) (width 0.25) (layer "F.Cu") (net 23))
 (segment (start 126.410829 78.92324) (end 125.72 79.614069) (width 0.25) (layer "F.Cu") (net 23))
 (segment (start 126.410829 78.92324) (end 126.410829 76.789171) (width 0.25) (layer "F.Cu") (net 23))
 (segment (start 125.72 85.65) (end 126.365 86.295) (width 0.25) (layer "F.Cu") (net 23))
 (segment (start 125.72 79.614069) (end 125.72 85.65) (width 0.25) (layer "F.Cu") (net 23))
 (segment (start 125.814158 76.1925) (end 125.75 76.1925) (width 0.25) (layer "F.Cu") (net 23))
 (segment (start 127.605829 78.92324) (end 127 79.529069) (width 0.25) (layer "F.Cu") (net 24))
 (segment (start 127 79.529069) (end 127 85.66) (width 0.25) (layer "F.Cu") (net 24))
 (segment (start 127.605829 76.805829) (end 128.219158 76.1925) (width 0.25) (layer "F.Cu") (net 24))
 (segment (start 127 85.66) (end 127.635 86.295) (width 0.25) (layer "F.Cu") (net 24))
 (segment (start 128.219158 76.1925) (end 128.25 76.1925) (width 0.25) (layer "F.Cu") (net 24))
 (segment (start 127.605829 78.92324) (end 127.605829 76.805829) (width 0.25) (layer "F.Cu") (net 24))
 (segment (start 143.51 85.853249) (end 143.51 86.23) (width 0.25) (layer "F.Cu") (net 19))
 (segment (start 142.586751 84.93) (end 143.51 85.853249) (width 0.25) (layer "F.Cu") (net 19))
 (segment (start 140.043857 77.218643) (end 140.043857 83.657106) (width 0.25) (layer "F.Cu") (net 19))
 (segment (start 141.07 76.1925) (end 140.043857 77.218643) (width 0.25) (layer "F.Cu") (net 19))
 (segment (start 141.316751 84.93) (end 142.586751 84.93) (width 0.25) (layer "F.Cu") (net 19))
 (segment (start 140.043857 83.657106) (end 141.316751 84.93) (width 0.25) (layer "F.Cu") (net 19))
 (segment (start 144.055 82.401751) (end 144.055 84.120305) (width 0.25) (layer "F.Cu") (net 20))
 (segment (start 144.055 84.120305) (end 144.78 84.845305) (width 0.25) (layer "F.Cu") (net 20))
 (segment (start 144.155 82.301751) (end 144.055 82.401751) (width 0.25) (layer "F.Cu") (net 20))
 (segment (start 144.155 76.7775) (end 144.155 82.301751) (width 0.25) (layer "F.Cu") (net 20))
 (segment (start 143.57 76.1925) (end 144.155 76.7775) (width 0.25) (layer "F.Cu") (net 20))
 (segment (start 144.78 84.845305) (end 144.78 86.23) (width 0.25) (layer "F.Cu") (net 20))
 (segment (start 146.07 76.1925) (end 146.675 76.7975) (width 0.25) (layer "F.Cu") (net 21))
 (segment (start 146.675 82.301751) (end 146.5 82.476751) (width 0.25) (layer "F.Cu") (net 21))
 (segment (start 146.5 82.476751) (end 146.5 85.78) (width 0.25) (layer "F.Cu") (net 21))
 (segment (start 146.675 76.7975) (end 146.675 82.301751) (width 0.25) (layer "F.Cu") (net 21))
 (segment (start 146.5 85.78) (end 146.05 86.23) (width 0.25) (layer "F.Cu") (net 21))
 (segment (start 148.045 84.120305) (end 147.32 84.845305) (width 0.25) (layer "F.Cu") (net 22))
 (segment (start 148.045 82.401751) (end 148.045 84.120305) (width 0.25) (layer "F.Cu") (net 22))
 (segment (start 148.57 76.1925) (end 147.945 76.8175) (width 0.25) (layer "F.Cu") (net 22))
 (segment (start 147.945 76.8175) (end 147.945 82.301751) (width 0.25) (layer "F.Cu") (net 22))
 (segment (start 147.945 82.301751) (end 148.045 82.401751) (width 0.25) (layer "F.Cu") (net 22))
 (segment (start 147.32 84.845305) (end 147.32 86.23) (width 0.25) (layer "F.Cu") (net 22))
 (segment (start 126.25 98.290661) (end 132.099339 104.14) (width 0.25) (layer "F.Cu") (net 7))
 (segment (start 126.25 96.669339) (end 126.25 98.290661) (width 0.25) (layer "F.Cu") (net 7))
 (segment (start 126.939339 95.98) (end 126.25 96.669339) (width 0.25) (layer "F.Cu") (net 7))
 (segment (start 127 95.98) (end 126.939339 95.98) (width 0.25) (layer "F.Cu") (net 7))
 (segment (start 141.49 103.035685) (end 141.49 102.195) (width 0.25) (layer "F.Cu") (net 7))
 (segment (start 132.099339 104.14) (end 140.385685 104.14) (width 0.25) (layer "F.Cu") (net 7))
 (segment (start 140.385685 104.14) (end 141.49 103.035685) (width 0.25) (layer "F.Cu") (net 7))
 (segment (start 134.980002 92.77) (end 136.565 92.77) (width 0.25) (layer "F.Cu") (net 10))
 (segment (start 128 93.98) (end 128.424999 93.555001) (width 0.25) (layer "F.Cu") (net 10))
 (segment (start 134.195001 93.555001) (end 134.980002 92.77) (width 0.25) (layer "F.Cu") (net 10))
 (segment (start 128.424999 93.555001) (end 134.195001 93.555001) (width 0.25) (layer "F.Cu") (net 10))
 (segment (start 139.49 91.685685) (end 139.49 90.845) (width 0.25) (layer "F.Cu") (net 11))
 (segment (start 138.880685 92.295) (end 139.49 91.685685) (width 0.25) (layer "F.Cu") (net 11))
 (segment (start 127 93.98) (end 127 93.37896) (width 0.25) (layer "F.Cu") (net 11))
 (segment (start 127 93.37896) (end 128.08396 92.295) (width 0.25) (layer "F.Cu") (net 11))
 (segment (start 128.08396 92.295) (end 138.880685 92.295) (width 0.25) (layer "F.Cu") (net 11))
 (segment (start 136.549587 96.785413) (end 136.565 96.77) (width 0.25) (layer "F.Cu") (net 17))
 (segment (start 134.086455 94.516554) (end 134.086455 96.705213) (width 0.25) (layer "F.Cu") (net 17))
 (segment (start 140.97 86.23) (end 140.97 87.841889) (width 0.25) (layer "F.Cu") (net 17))
 (segment (start 134.006255 96.785413) (end 136.549587 96.785413) (width 0.25) (layer "F.Cu") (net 17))
 (segment (start 134.086455 96.705213) (end 134.006255 96.785413) (width 0.25) (layer "F.Cu") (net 17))
 (segment (start 140.97 87.841889) (end 141.296857 88.168746) (width 0.25) (layer "F.Cu") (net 17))
 (via (at 141.296857 88.168746) (size 0.8) (drill 0.4) (layers "F.Cu" "B.Cu") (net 17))
 (via (at 134.086455 94.516554) (size 0.8) (drill 0.4) (layers "F.Cu" "B.Cu") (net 17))
 (segment (start 141.296857 88.168746) (end 140.565603 88.9) (width 0.25) (layer "B.Cu") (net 17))
 (segment (start 140.565603 88.9) (end 137.16 88.9) (width 0.25) (layer "B.Cu") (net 17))
 (segment (start 134.086455 91.973545) (end 134.086455 94.516554) (width 0.25) (layer "B.Cu") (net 17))
 (segment (start 137.16 88.9) (end 134.086455 91.973545) (width 0.25) (layer "B.Cu") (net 17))
 (segment (start 132.145 81.345) (end 139.99 89.19) (width 0.25) (layer "F.Cu") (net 25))
 (segment (start 128.905 81.345) (end 132.145 81.345) (width 0.25) (layer "F.Cu") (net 25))
 (segment (start 139.99 89.19) (end 139.99 90.845) (width 0.25) (layer "F.Cu") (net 25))
 (segment (start 139.416844 87.748508) (end 140.49 88.821664) (width 0.25) (layer "F.Cu") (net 26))
 (segment (start 137.16 83.82) (end 139.416844 86.076844) (width 0.25) (layer "F.Cu") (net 26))
 (segment (start 139.416844 86.076844) (end 139.416844 87.748508) (width 0.25) (layer "F.Cu") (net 26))
 (segment (start 125.095 81.234246) (end 123.779562 79.918808) (width 0.25) (layer "F.Cu") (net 26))
 (segment (start 125.095 81.345) (end 125.095 81.234246) (width 0.25) (layer "F.Cu") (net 26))
 (segment (start 140.49 88.821664) (end 140.49 90.845) (width 0.25) (layer "F.Cu") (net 26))
 (via (at 137.16 83.82) (size 0.8) (drill 0.4) (layers "F.Cu" "B.Cu") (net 26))
 (via (at 123.779562 79.918808) (size 0.8) (drill 0.4) (layers "F.Cu" "B.Cu") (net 26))
 (segment (start 123.779562 79.918808) (end 125.59148 78.10689) (width 0.25) (layer "B.Cu") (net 26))
 (segment (start 131.44689 78.10689) (end 137.16 83.82) (width 0.25) (layer "B.Cu") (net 26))
 (segment (start 125.59148 78.10689) (end 131.44689 78.10689) (width 0.25) (layer "B.Cu") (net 26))
 (segment (start 134.05 91.44) (end 137.16 91.44) (width 0.25) (layer "F.Cu") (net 28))
 (segment (start 140.99 92.73) (end 140.99 90.845) (width 0.25) (layer "F.Cu") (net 28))
 (segment (start 128.905 86.295) (end 134.05 91.44) (width 0.25) (layer "F.Cu") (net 28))
 (segment (start 142.24 93.98) (end 140.99 92.73) (width 0.25) (layer "F.Cu") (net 28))
 (via (at 142.24 93.98) (size 0.8) (drill 0.4) (layers "F.Cu" "B.Cu") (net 28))
 (via (at 137.16 91.44) (size 0.8) (drill 0.4) (layers "F.Cu" "B.Cu") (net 28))
 (segment (start 137.16 91.44) (end 139.7 93.98) (width 0.25) (layer "B.Cu") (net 28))
 (segment (start 139.7 93.98) (end 142.24 93.98) (width 0.25) (layer "B.Cu") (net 28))
 (segment (start 147.32 83.82) (end 147.32 81.28) (width 0.25) (layer "F.Cu") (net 12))
 (segment (start 145.99 90.845) (end 145.99 90.23) (width 0.25) (layer "F.Cu") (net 12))
 (segment (start 145.99 90.23) (end 147.32 88.9) (width 0.25) (layer "F.Cu") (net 12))
 (via (at 147.32 88.9) (size 0.8) (drill 0.4) (layers "F.Cu" "B.Cu") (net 12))
 (via (at 147.32 83.82) (size 0.8) (drill 0.4) (layers "F.Cu" "B.Cu") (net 12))
 (segment (start 147.32 88.9) (end 147.32 83.82) (width 0.25) (layer "B.Cu") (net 12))
 (segment (start 145.5045 84.526755) (end 146.05 83.981255) (width 0.25) (layer "F.Cu") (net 13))
 (segment (start 146.05 83.981255) (end 146.05 81.28) (width 0.25) (layer "F.Cu") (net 13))
 (segment (start 145.49 89.189503) (end 145.779503 88.9) (width 0.25) (layer "F.Cu") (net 13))
 (segment (start 145.49 90.845) (end 145.49 89.189503) (width 0.25) (layer "F.Cu") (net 13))
 (via (at 145.5045 84.526755) (size 0.8) (drill 0.4) (layers "F.Cu" "B.Cu") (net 13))
 (via (at 145.779503 88.9) (size 0.8) (drill 0.4) (layers "F.Cu" "B.Cu") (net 13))
 (segment (start 145.779503 88.9) (end 145.779503 84.801758) (width 0.25) (layer "B.Cu") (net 13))
 (segment (start 145.779503 84.801758) (end 145.5045 84.526755) (width 0.25) (layer "B.Cu") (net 13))
 (segment (start 144.78 83.82) (end 144.78 81.28) (width 0.25) (layer "F.Cu") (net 14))
 (segment (start 144.99 90.845) (end 144.99 89.11) (width 0.25) (layer "F.Cu") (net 14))
 (segment (start 144.99 89.11) (end 144.78 88.9) (width 0.25) (layer "F.Cu") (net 14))
 (via (at 144.78 88.9) (size 0.8) (drill 0.4) (layers "F.Cu" "B.Cu") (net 14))
 (via (at 144.78 83.82) (size 0.8) (drill 0.4) (layers "F.Cu" "B.Cu") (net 14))
 (segment (start 144.78 88.9) (end 144.78 83.82) (width 0.25) (layer "B.Cu") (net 14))
 (segment (start 142.24 83.82) (end 142.24 83.580355) (width 0.25) (layer "F.Cu") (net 15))
 (segment (start 143.51 82.310355) (end 143.51 81.28) (width 0.25) (layer "F.Cu") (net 15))
 (segment (start 144.49 90.845) (end 144.49 90.00119) (width 0.25) (layer "F.Cu") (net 15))
 (segment (start 142.24 83.580355) (end 143.51 82.310355) (width 0.25) (layer "F.Cu") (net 15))
 (segment (start 144.49 90.00119) (end 143.95931 89.4705) (width 0.25) (layer "F.Cu") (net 15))
 (via (at 142.24 83.82) (size 0.8) (drill 0.4) (layers "F.Cu" "B.Cu") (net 15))
 (via (at 143.95931 89.4705) (size 0.8) (drill 0.4) (layers "F.Cu" "B.Cu") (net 15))
 (segment (start 143.95931 89.4705) (end 142.24 87.75119) (width 0.25) (layer "B.Cu") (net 15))
 (segment (start 142.24 87.75119) (end 142.24 83.82) (width 0.25) (layer "B.Cu") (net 15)))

